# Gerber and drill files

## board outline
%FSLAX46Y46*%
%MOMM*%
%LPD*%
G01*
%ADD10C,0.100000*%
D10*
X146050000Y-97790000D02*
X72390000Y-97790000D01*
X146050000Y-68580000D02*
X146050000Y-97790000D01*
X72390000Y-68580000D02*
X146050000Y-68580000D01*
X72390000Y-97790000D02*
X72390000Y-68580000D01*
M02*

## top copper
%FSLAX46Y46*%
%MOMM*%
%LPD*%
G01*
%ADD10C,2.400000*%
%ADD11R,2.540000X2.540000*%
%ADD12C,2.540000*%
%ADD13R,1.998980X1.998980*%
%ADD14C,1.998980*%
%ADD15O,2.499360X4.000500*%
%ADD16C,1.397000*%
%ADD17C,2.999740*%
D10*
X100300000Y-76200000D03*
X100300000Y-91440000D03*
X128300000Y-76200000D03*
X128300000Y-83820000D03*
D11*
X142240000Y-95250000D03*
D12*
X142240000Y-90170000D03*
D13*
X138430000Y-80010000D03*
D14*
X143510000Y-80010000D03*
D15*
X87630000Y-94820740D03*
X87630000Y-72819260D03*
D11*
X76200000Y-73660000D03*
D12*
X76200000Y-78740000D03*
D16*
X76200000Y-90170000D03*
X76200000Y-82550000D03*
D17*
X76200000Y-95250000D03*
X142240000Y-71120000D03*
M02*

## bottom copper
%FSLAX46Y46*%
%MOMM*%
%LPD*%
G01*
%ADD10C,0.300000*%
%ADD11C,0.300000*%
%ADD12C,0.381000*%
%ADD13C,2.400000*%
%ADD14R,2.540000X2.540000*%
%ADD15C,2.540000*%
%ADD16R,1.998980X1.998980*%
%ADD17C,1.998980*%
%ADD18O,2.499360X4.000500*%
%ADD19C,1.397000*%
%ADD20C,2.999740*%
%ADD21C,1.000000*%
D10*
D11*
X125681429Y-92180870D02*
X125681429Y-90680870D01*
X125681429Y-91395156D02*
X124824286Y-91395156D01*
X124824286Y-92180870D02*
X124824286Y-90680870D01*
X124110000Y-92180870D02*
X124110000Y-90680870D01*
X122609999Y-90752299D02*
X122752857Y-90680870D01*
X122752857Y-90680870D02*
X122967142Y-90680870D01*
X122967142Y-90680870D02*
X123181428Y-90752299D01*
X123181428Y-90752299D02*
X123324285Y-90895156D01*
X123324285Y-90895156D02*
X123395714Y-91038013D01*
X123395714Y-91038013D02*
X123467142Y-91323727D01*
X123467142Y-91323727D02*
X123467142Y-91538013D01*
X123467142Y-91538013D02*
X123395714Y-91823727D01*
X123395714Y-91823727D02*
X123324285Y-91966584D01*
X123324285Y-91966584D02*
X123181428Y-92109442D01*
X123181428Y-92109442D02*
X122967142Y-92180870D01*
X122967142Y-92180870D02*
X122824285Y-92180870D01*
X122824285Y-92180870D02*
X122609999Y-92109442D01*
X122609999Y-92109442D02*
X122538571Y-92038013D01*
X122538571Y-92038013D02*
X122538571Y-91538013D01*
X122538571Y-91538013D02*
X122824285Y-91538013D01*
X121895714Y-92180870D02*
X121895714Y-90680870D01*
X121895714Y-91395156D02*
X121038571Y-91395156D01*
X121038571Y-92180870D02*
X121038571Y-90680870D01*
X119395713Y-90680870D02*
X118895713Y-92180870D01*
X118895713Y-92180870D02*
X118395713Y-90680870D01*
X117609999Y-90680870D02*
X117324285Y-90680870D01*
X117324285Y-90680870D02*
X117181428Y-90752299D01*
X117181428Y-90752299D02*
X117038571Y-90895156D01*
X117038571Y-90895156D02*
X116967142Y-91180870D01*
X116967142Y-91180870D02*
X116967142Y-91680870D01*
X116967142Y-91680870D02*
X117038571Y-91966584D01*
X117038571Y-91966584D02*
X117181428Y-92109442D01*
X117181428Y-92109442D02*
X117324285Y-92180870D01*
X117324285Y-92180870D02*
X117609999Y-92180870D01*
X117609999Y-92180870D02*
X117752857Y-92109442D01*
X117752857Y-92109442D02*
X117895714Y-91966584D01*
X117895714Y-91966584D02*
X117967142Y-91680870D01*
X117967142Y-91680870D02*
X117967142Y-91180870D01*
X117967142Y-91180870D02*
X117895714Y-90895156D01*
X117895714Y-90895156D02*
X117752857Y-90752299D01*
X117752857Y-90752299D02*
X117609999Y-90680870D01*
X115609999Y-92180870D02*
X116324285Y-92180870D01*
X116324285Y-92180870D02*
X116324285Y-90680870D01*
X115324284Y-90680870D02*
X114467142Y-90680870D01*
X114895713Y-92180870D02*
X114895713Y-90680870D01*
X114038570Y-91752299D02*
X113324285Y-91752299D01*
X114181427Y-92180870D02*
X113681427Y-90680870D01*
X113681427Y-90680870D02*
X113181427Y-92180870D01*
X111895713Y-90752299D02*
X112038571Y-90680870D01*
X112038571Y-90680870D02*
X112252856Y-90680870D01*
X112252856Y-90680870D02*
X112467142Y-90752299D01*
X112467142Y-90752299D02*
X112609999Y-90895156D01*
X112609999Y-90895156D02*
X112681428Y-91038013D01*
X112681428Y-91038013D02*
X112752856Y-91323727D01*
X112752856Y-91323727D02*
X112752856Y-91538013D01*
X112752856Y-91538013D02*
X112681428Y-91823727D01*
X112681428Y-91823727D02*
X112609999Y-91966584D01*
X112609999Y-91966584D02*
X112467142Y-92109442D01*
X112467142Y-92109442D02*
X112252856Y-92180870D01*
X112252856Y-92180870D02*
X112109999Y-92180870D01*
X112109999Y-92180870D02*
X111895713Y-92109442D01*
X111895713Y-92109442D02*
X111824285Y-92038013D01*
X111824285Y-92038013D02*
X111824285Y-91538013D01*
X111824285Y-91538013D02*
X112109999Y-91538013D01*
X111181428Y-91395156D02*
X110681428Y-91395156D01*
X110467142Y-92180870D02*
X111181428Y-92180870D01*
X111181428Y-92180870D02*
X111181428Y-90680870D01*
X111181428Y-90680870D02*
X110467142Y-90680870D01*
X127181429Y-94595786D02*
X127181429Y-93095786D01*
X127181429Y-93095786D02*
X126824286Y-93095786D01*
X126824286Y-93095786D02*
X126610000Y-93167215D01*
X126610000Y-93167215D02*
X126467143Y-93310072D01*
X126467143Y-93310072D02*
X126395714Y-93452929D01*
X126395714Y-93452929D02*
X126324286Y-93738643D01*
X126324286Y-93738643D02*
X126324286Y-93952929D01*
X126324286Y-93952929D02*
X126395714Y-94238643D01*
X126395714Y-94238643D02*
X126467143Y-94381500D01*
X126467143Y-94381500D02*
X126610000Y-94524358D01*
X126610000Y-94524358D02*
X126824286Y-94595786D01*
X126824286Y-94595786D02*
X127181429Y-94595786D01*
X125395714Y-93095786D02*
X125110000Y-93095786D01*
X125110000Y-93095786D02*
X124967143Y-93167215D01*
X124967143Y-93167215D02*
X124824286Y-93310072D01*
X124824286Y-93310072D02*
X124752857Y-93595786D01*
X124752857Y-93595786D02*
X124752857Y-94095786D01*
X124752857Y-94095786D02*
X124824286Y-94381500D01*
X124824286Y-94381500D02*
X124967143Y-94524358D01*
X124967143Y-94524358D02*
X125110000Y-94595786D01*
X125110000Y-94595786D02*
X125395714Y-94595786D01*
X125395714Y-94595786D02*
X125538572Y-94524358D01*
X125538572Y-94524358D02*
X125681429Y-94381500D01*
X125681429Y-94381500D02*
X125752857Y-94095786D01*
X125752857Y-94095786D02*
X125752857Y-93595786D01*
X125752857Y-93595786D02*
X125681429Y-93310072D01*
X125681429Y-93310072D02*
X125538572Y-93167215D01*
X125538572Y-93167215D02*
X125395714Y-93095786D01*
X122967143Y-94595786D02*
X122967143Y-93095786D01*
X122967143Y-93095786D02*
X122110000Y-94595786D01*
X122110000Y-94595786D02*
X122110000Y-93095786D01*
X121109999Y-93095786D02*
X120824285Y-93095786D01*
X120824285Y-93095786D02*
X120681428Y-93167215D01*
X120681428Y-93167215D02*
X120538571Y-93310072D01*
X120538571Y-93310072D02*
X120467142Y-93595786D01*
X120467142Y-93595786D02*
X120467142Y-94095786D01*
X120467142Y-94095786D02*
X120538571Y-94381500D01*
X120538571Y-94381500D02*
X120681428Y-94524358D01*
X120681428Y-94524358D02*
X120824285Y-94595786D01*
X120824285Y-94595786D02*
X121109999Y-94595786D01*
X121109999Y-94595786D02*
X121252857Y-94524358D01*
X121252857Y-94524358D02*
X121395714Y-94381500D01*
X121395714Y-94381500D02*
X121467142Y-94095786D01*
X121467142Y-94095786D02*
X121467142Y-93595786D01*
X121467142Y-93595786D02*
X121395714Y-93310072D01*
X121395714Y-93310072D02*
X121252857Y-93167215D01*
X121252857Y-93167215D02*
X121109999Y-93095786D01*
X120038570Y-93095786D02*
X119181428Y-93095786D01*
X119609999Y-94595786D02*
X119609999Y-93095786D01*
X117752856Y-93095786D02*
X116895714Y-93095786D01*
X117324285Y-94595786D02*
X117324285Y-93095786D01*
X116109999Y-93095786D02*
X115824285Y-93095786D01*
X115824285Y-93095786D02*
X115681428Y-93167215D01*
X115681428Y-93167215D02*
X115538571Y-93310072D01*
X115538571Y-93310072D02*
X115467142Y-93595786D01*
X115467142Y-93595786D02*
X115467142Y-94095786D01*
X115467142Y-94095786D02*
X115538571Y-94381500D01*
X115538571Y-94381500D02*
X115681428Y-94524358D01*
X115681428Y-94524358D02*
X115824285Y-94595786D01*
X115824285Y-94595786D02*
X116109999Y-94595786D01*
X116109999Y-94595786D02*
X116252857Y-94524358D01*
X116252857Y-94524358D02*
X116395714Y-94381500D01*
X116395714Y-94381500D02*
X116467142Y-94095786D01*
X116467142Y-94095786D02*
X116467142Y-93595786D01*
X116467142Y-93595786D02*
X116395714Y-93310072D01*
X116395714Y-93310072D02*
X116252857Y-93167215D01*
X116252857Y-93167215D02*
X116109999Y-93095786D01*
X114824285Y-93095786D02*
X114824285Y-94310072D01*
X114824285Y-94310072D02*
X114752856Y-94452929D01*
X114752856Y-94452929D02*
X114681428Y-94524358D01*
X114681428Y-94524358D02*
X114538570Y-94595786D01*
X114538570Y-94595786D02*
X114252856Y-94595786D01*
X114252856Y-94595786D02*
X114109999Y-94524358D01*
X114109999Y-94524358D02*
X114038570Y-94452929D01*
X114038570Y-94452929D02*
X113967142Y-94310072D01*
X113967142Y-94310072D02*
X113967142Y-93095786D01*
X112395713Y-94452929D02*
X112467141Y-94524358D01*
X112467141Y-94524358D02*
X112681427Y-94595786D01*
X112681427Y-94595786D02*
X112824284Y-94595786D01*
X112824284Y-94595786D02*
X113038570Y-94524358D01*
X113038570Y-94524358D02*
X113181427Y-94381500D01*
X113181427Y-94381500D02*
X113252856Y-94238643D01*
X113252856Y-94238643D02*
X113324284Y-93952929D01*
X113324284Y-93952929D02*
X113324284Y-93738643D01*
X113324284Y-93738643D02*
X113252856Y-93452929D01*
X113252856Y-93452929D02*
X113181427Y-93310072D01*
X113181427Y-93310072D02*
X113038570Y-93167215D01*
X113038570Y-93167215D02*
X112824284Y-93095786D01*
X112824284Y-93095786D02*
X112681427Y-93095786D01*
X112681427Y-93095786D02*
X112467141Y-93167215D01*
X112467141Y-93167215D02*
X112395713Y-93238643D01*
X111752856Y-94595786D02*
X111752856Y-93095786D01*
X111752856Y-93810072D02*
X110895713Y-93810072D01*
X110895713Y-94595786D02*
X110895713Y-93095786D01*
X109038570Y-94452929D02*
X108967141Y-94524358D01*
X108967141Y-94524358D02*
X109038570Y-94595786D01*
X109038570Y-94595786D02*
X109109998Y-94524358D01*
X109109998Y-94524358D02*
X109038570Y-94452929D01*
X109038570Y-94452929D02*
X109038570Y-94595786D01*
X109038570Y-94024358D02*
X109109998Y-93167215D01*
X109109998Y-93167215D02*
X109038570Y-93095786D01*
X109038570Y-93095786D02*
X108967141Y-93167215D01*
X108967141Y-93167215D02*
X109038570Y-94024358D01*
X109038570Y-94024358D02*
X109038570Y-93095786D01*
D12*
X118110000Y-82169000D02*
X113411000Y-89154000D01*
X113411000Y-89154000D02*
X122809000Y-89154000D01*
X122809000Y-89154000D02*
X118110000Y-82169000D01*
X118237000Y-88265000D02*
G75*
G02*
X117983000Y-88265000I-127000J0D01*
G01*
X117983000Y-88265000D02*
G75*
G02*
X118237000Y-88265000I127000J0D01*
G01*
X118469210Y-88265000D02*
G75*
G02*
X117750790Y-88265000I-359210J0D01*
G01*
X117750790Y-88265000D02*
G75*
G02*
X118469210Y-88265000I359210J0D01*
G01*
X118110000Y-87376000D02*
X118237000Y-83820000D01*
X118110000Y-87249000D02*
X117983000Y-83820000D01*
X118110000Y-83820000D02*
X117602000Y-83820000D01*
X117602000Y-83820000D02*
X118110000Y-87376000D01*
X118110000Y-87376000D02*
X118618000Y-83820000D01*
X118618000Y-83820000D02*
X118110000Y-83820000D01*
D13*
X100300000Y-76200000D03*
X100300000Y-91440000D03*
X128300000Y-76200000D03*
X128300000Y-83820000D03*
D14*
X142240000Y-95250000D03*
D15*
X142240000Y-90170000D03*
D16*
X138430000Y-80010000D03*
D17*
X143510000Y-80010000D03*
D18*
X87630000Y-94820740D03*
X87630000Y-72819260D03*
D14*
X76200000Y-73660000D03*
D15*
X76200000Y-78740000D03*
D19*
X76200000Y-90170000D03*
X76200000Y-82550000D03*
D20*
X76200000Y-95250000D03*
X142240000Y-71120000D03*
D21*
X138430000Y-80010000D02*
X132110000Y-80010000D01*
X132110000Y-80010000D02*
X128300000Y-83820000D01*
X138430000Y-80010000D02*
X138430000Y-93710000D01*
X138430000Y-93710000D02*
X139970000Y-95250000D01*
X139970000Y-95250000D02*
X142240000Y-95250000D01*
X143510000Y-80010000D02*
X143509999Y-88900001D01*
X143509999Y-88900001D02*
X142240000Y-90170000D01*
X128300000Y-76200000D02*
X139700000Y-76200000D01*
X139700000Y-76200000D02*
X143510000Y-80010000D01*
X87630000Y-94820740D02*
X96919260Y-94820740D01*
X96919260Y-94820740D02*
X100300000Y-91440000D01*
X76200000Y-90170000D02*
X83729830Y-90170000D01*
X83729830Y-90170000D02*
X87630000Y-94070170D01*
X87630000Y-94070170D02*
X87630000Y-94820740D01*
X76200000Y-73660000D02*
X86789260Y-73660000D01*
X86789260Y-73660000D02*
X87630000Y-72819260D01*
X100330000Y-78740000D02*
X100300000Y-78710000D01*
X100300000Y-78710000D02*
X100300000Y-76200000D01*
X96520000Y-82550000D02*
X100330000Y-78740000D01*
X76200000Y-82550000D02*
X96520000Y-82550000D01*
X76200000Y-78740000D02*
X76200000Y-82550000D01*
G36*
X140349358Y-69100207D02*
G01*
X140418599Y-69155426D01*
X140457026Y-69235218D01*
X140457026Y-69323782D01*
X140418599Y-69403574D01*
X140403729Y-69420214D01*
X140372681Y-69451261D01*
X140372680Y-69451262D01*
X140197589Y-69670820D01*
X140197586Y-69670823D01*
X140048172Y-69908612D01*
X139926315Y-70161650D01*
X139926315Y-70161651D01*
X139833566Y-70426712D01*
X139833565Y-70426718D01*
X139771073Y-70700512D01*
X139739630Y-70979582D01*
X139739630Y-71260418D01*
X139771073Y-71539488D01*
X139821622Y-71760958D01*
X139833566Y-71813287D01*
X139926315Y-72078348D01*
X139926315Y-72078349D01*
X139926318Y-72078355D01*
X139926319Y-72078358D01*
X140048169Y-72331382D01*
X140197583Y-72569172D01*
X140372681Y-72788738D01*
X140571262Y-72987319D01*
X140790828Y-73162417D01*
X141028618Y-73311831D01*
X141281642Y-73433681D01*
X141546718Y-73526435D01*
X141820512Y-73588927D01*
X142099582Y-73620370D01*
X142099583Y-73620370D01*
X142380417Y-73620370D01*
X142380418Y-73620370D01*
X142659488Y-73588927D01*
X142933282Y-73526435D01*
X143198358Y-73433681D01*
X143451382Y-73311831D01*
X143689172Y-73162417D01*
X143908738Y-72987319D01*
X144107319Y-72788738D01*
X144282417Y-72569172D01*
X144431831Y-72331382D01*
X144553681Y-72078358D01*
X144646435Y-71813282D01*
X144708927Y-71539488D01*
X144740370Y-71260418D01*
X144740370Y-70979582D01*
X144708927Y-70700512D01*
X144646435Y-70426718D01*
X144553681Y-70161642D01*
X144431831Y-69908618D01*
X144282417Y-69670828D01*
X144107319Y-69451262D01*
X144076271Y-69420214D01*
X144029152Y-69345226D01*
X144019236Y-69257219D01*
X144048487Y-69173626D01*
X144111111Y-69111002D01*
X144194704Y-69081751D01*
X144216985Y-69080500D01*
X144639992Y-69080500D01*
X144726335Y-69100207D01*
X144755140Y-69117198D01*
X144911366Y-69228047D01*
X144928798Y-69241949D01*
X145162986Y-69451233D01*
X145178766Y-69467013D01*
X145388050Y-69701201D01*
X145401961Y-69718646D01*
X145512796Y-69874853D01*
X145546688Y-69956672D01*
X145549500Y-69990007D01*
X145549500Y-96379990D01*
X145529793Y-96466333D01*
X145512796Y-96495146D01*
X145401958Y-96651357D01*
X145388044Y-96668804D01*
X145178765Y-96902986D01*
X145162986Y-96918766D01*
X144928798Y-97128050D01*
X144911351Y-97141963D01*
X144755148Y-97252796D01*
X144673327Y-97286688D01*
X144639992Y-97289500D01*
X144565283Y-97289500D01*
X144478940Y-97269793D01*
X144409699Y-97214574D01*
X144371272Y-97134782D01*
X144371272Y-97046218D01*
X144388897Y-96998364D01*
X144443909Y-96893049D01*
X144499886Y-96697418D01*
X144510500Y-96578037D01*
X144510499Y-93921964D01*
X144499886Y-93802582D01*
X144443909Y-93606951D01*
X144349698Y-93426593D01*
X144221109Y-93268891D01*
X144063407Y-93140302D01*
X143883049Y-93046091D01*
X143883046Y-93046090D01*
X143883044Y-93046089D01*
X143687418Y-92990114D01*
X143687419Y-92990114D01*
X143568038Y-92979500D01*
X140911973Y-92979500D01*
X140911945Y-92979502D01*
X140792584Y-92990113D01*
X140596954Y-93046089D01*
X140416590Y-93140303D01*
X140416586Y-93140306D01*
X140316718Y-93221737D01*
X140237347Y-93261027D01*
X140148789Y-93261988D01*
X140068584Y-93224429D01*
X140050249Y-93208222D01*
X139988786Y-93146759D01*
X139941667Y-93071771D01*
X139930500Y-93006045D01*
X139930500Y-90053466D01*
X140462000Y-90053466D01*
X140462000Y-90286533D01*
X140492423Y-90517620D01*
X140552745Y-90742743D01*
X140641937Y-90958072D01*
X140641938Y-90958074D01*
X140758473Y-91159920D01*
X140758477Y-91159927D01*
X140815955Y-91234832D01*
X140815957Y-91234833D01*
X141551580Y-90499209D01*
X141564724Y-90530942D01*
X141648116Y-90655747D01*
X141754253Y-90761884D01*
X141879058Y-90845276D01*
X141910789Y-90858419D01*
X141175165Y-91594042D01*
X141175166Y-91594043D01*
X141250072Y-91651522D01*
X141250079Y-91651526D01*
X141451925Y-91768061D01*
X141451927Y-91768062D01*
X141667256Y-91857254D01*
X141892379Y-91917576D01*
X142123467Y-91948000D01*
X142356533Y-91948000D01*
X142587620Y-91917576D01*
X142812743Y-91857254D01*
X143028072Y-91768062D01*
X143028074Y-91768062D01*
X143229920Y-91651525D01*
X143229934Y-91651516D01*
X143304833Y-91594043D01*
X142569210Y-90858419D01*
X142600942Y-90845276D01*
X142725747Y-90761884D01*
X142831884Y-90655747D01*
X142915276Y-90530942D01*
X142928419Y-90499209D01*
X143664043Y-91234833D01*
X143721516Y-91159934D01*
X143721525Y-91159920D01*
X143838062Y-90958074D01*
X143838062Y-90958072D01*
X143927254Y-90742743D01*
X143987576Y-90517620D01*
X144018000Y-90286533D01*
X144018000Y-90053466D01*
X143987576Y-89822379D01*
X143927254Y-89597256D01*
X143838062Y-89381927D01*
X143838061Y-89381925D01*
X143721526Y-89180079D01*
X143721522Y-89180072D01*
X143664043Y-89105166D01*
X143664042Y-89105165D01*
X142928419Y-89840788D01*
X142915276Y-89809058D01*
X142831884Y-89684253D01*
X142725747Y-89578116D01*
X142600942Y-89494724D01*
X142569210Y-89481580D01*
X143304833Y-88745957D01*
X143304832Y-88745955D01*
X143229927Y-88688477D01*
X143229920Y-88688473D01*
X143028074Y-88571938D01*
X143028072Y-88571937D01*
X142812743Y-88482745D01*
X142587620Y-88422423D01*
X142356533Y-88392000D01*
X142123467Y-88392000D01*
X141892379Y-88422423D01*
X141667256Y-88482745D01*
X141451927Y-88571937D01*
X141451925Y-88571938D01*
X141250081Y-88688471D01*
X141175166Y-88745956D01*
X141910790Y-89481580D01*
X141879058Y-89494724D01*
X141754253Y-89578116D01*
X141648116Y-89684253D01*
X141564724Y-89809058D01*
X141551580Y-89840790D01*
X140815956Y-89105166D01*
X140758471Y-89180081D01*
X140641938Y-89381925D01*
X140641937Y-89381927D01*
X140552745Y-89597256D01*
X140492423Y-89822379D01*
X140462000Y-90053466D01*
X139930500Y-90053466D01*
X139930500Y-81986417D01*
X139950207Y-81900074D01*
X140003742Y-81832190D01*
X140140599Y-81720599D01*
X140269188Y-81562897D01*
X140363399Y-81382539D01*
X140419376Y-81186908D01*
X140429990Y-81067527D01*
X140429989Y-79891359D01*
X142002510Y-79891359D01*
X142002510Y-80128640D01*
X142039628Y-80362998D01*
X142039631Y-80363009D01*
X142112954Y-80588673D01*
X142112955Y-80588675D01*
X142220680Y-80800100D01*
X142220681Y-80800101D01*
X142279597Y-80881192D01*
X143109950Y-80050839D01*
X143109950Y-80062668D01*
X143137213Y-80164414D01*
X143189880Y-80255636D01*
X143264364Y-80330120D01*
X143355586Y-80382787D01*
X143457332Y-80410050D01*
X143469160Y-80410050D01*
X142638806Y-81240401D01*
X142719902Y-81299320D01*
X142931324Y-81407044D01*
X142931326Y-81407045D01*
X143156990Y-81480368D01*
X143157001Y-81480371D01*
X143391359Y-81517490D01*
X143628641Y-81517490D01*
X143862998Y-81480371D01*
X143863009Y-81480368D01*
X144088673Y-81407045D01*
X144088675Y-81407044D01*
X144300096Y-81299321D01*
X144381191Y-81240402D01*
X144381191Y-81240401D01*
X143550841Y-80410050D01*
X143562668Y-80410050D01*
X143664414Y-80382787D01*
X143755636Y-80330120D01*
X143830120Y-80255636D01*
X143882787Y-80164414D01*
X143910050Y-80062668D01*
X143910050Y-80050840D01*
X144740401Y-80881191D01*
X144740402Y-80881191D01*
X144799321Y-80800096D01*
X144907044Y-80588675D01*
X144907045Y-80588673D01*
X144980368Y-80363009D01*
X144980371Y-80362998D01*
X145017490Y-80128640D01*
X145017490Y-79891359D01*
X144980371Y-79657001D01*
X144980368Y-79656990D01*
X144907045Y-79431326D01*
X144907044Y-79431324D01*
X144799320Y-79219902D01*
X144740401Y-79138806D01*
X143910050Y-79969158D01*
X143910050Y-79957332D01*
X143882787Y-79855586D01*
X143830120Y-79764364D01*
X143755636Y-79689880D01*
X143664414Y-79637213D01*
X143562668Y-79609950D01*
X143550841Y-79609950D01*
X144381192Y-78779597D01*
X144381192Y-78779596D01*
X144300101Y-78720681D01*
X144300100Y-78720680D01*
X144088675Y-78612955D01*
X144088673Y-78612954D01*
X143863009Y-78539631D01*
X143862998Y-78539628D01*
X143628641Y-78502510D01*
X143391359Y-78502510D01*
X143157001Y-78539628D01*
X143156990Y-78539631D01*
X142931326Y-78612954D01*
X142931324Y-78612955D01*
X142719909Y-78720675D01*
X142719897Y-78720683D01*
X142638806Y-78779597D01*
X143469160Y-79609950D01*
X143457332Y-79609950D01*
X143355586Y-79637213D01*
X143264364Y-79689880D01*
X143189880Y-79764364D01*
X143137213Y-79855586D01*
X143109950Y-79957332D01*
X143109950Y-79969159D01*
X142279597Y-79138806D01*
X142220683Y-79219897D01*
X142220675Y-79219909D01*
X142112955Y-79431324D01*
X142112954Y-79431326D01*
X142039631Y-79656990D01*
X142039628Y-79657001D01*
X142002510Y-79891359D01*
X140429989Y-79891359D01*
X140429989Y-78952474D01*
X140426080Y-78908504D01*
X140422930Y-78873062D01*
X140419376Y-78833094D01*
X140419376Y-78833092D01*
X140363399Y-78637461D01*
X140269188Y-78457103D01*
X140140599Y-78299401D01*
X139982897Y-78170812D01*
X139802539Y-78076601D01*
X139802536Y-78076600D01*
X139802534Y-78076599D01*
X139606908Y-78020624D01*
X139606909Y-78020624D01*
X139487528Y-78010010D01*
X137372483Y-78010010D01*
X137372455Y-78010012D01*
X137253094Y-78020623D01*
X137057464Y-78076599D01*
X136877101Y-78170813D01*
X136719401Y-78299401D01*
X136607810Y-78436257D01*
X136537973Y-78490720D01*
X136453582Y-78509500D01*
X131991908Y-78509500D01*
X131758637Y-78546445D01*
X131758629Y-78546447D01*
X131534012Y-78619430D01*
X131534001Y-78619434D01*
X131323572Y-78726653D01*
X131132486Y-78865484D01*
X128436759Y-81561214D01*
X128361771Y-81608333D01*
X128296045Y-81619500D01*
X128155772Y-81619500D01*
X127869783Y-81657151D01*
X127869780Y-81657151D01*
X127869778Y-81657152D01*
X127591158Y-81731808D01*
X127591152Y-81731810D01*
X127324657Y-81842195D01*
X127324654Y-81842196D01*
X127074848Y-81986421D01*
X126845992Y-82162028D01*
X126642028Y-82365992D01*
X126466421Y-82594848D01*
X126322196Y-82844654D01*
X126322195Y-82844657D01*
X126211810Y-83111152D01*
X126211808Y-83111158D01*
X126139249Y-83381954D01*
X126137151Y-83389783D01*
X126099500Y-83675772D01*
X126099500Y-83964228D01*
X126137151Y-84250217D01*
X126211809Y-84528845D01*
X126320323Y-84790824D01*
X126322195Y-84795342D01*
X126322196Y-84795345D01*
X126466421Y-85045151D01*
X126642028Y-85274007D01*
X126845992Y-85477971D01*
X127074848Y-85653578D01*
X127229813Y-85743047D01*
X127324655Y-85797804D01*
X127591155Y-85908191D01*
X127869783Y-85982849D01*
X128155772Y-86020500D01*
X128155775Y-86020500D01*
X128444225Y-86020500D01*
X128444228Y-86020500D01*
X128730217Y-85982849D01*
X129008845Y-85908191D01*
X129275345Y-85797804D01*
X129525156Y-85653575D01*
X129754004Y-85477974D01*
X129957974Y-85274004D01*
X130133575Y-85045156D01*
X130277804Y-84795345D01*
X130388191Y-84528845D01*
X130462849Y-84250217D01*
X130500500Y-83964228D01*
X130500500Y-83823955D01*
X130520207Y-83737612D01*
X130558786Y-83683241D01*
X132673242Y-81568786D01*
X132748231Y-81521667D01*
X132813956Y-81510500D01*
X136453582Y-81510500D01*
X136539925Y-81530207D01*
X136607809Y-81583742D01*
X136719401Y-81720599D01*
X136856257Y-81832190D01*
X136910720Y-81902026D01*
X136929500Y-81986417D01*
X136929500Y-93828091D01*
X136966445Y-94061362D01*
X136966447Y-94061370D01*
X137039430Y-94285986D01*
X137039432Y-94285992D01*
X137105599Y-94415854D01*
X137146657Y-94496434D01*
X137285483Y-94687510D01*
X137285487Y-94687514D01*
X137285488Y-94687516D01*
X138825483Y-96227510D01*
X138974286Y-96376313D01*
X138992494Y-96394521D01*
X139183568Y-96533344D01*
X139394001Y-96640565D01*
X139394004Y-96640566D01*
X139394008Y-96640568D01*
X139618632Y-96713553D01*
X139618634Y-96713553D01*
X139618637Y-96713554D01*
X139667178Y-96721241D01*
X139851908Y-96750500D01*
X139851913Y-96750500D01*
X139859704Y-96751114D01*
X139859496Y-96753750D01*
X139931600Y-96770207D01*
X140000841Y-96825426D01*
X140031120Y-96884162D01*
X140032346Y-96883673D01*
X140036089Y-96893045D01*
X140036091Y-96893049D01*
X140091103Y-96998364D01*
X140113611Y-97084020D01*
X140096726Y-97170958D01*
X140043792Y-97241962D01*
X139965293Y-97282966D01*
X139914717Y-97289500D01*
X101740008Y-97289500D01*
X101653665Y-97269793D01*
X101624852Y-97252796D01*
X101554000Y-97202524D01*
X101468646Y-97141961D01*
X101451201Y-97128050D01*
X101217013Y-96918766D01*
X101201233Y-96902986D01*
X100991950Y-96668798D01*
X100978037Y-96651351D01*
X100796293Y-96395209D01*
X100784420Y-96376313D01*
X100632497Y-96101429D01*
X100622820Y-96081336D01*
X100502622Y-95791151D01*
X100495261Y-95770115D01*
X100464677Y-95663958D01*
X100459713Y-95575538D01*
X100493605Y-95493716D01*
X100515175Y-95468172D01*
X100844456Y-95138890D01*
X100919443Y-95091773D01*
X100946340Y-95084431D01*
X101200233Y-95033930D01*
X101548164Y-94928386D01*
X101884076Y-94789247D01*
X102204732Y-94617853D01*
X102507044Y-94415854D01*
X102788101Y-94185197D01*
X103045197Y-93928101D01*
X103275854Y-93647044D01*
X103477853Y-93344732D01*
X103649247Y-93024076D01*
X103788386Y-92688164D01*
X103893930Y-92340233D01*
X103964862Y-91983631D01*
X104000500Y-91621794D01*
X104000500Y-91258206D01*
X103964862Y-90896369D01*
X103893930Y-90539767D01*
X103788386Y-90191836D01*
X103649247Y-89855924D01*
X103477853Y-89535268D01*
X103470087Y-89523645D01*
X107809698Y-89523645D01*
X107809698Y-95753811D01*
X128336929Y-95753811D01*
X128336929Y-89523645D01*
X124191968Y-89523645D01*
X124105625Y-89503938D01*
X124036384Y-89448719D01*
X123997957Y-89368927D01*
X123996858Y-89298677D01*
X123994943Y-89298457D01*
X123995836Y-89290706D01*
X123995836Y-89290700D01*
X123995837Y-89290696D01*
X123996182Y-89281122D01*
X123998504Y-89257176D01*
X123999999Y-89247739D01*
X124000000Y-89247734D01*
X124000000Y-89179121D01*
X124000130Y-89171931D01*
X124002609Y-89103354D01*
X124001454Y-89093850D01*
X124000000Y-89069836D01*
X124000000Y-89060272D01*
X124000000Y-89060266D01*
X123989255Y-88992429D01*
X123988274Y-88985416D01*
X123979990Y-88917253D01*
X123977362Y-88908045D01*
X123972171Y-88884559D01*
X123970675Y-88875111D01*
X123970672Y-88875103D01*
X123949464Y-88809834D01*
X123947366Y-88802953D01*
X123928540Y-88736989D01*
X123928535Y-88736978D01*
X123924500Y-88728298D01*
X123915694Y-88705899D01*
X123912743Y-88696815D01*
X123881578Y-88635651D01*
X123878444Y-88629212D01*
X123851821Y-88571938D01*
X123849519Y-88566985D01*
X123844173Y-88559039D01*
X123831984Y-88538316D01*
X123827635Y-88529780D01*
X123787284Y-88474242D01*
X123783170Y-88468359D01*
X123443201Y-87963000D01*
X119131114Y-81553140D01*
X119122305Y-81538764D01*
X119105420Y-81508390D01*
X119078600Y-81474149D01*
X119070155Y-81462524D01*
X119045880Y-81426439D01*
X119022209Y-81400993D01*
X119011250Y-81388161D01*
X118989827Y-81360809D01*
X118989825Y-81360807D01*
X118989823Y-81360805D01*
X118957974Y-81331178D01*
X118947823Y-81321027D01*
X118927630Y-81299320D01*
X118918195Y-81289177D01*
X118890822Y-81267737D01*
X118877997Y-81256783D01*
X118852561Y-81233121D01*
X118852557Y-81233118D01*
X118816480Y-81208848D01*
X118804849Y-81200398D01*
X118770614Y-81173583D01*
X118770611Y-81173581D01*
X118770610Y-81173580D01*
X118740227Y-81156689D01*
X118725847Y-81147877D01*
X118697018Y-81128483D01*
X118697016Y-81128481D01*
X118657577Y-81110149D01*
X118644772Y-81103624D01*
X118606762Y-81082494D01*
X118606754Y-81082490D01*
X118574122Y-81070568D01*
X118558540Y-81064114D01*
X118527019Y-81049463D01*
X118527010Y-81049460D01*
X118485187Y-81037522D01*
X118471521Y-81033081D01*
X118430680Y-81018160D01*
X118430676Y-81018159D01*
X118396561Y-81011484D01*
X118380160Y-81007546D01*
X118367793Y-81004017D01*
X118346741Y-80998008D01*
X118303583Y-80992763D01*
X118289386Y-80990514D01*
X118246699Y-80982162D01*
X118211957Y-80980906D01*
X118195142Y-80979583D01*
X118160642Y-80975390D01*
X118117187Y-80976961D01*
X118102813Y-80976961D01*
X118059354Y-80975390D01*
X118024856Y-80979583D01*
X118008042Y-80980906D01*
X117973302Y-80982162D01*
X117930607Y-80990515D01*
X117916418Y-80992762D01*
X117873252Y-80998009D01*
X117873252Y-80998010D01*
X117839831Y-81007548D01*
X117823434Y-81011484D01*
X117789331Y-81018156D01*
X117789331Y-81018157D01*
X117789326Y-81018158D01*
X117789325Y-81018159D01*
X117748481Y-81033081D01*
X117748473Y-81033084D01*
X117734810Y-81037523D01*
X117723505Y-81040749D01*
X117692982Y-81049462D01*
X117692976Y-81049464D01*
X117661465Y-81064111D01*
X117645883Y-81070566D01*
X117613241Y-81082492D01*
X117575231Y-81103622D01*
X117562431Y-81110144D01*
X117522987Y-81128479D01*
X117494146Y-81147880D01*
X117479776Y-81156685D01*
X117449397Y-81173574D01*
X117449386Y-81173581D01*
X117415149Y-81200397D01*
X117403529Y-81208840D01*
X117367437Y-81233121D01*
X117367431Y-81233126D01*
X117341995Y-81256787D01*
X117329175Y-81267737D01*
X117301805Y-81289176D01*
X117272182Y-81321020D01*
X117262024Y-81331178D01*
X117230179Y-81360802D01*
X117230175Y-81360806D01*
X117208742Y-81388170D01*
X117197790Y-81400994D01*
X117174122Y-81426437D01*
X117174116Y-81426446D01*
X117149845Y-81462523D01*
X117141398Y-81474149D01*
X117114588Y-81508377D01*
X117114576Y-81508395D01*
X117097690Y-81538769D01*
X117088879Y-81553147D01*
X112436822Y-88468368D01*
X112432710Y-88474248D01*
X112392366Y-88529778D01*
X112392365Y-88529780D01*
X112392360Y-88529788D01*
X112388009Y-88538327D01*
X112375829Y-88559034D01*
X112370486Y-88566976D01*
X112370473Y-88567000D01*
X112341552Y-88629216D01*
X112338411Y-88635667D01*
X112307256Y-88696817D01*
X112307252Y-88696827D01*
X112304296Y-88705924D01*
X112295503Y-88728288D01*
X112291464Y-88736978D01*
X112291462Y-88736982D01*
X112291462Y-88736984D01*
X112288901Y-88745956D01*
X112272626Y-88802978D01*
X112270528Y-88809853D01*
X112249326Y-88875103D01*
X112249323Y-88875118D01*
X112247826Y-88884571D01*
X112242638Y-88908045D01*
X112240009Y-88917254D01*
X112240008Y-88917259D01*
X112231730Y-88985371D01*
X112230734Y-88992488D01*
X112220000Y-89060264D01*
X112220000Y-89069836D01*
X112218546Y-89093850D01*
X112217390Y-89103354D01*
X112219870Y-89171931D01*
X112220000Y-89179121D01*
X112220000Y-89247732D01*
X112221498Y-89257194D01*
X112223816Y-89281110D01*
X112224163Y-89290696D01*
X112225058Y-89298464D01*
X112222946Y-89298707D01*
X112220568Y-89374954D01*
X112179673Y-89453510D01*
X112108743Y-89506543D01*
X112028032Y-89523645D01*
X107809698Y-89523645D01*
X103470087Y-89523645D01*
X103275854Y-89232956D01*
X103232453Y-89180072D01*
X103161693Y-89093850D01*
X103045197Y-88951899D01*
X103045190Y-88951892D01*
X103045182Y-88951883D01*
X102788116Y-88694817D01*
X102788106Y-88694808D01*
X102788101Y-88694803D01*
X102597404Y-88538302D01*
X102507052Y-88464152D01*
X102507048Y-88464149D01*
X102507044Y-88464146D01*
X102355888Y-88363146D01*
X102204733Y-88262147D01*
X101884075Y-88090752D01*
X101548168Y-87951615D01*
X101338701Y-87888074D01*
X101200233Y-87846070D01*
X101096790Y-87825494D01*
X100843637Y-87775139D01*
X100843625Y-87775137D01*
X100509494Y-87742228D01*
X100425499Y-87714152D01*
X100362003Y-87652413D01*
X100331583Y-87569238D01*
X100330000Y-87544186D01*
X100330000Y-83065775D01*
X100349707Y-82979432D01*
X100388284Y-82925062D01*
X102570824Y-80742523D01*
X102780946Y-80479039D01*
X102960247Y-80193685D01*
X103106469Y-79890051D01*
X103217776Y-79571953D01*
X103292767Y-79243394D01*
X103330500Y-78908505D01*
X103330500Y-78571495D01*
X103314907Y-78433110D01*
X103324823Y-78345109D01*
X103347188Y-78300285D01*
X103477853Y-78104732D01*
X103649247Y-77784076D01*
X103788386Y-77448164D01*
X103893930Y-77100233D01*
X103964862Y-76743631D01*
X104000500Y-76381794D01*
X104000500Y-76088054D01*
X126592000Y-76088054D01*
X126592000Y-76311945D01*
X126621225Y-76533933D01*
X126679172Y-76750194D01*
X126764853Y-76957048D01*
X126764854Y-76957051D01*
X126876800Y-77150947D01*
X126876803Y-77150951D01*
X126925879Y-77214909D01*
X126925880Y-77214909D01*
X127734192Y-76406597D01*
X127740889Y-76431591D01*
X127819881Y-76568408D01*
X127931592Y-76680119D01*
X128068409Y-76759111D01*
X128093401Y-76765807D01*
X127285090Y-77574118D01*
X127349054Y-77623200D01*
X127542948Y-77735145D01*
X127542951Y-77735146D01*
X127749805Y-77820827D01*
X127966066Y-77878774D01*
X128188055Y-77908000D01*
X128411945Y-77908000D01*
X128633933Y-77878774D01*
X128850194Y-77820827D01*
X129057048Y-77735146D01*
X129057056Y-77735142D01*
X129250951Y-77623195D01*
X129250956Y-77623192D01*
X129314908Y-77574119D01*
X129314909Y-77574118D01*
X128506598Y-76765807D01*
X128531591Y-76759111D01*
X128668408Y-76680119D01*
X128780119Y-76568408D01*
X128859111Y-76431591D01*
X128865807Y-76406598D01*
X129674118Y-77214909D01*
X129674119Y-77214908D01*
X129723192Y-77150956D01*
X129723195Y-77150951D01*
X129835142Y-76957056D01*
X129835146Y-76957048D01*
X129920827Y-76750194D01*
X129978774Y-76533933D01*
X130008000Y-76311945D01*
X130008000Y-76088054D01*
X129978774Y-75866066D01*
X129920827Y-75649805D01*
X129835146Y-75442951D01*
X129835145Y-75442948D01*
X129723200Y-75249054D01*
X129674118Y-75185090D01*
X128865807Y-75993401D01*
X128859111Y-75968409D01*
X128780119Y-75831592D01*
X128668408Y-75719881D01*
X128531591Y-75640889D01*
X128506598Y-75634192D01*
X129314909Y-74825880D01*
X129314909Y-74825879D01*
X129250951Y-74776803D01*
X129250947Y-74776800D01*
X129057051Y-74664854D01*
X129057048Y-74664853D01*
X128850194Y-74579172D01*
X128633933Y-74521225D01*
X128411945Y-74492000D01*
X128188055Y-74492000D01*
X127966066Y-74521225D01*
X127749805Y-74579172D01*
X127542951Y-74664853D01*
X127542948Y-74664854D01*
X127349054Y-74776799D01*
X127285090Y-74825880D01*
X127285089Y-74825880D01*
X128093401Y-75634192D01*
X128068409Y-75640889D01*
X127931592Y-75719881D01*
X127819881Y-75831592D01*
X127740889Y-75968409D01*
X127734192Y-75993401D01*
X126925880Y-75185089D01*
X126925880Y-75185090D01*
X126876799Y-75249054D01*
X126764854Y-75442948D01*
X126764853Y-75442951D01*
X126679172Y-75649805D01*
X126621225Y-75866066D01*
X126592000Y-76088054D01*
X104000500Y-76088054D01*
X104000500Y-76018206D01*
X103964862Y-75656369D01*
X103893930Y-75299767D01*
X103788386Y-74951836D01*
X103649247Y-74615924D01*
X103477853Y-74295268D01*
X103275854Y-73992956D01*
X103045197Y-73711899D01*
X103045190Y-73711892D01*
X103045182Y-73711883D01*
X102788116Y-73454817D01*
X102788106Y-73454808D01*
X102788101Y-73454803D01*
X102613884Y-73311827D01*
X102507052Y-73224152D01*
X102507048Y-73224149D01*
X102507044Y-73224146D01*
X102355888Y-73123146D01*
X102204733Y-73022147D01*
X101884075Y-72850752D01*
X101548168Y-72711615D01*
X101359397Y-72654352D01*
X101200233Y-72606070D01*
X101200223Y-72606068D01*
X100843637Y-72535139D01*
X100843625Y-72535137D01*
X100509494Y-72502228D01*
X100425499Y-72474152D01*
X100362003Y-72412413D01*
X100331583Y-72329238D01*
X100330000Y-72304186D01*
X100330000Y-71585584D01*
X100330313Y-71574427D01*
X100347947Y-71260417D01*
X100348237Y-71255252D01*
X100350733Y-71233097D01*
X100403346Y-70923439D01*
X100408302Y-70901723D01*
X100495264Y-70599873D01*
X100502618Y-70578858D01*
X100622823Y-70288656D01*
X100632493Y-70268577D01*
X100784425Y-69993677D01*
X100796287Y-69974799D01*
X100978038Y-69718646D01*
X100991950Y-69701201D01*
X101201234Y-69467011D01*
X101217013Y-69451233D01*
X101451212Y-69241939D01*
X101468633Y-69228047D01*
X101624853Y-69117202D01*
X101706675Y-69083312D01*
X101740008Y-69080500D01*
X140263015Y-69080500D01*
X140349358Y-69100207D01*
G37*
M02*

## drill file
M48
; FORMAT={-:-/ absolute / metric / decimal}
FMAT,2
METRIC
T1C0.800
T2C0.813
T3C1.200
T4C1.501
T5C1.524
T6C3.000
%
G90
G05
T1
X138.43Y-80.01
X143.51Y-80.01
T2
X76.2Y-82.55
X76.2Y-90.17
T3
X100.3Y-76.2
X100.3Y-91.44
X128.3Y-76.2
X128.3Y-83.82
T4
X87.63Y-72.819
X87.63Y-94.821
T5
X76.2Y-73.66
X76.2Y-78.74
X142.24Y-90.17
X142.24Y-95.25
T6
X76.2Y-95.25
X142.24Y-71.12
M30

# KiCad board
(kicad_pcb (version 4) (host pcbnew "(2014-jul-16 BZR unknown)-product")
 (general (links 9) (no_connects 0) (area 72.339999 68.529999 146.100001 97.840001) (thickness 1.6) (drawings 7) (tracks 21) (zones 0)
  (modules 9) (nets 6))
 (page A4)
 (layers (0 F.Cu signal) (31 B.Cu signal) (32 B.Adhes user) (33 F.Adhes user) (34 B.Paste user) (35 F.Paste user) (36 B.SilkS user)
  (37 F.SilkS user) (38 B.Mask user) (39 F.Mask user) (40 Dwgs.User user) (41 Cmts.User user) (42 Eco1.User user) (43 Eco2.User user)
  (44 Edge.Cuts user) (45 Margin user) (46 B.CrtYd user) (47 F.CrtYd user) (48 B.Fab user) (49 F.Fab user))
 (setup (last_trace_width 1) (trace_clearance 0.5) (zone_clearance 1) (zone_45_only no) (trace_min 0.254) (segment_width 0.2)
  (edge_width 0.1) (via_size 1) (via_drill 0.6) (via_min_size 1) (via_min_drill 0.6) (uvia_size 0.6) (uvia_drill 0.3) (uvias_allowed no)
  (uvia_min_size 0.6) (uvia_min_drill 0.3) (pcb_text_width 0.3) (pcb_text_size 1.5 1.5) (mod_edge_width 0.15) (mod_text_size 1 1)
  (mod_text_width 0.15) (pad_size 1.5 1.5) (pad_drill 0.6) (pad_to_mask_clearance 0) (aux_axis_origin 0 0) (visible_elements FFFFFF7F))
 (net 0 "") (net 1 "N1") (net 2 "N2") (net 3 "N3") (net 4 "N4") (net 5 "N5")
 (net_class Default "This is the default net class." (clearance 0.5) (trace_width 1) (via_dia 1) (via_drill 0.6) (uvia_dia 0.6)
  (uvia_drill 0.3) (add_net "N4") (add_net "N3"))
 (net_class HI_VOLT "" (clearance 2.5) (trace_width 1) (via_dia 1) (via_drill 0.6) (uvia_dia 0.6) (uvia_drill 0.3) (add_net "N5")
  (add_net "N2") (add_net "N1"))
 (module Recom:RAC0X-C (layer F.Cu) (at 114.3 83.82)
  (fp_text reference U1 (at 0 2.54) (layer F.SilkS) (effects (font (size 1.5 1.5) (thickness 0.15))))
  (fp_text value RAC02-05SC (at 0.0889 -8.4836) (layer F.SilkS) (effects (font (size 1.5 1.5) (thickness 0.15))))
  (pad 1 thru_hole circle (at -14 -7.62) (size 2.4 2.4) (drill 1.2) (layers *.Cu *.Mask F.SilkS) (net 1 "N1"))
  (pad 2 thru_hole circle (at -14 7.62) (size 2.4 2.4) (drill 1.2) (layers *.Cu *.Mask F.SilkS) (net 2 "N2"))
  (pad 3 thru_hole circle (at 14 -7.62) (size 2.4 2.4) (drill 1.2) (layers *.Cu *.Mask F.SilkS) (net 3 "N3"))
  (pad 4 thru_hole circle (at 14 0) (size 2.4 2.4) (drill 1.2) (layers *.Cu *.Mask F.SilkS) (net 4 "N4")))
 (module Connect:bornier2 (layer F.Cu) (at 142.24 92.71 90)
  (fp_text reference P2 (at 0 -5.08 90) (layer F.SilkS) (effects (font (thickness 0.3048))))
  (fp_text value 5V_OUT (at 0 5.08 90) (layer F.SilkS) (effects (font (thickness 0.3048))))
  (pad 1 thru_hole rect (at -2.54 0 90) (size 2.54 2.54) (drill 1.524) (layers *.Cu *.Mask F.SilkS) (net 4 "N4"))
  (pad 2 thru_hole circle (at 2.54 0 90) (size 2.54 2.54) (drill 1.524) (layers *.Cu *.Mask F.SilkS) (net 3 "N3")))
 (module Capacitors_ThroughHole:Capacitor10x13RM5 (layer F.Cu) (at 140.97 80.01 270)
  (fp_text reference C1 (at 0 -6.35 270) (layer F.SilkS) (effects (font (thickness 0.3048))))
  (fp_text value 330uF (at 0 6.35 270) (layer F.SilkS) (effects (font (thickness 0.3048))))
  (pad 1 thru_hole rect (at 0 2.54 270) (size 1.99898 1.99898) (drill 0.8001) (layers *.Cu *.Mask F.SilkS) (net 4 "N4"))
  (pad 2 thru_hole circle (at 0 -2.54 270) (size 1.99898 1.99898) (drill 0.8001) (layers *.Cu *.Mask F.SilkS) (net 3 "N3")))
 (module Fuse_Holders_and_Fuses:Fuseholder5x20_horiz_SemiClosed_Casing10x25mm (layer F.Cu) (at 87.63 83.82 270)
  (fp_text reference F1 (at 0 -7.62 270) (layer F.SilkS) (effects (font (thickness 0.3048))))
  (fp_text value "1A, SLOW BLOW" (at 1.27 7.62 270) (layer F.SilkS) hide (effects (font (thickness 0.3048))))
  (pad 2 thru_hole oval (at 11.00074 0 180) (size 2.49936 4.0005) (drill 1.50114) (layers *.Cu *.Mask F.SilkS) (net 2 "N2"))
  (pad 1 thru_hole oval (at -11.00074 0 180) (size 2.49936 4.0005) (drill 1.50114) (layers *.Cu *.Mask F.SilkS) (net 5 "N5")))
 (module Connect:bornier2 (layer F.Cu) (at 76.2 76.2 270)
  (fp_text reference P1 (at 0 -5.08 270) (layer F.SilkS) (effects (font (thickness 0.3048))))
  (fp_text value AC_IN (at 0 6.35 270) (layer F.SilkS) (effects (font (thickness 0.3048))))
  (pad 1 thru_hole rect (at -2.54 0 270) (size 2.54 2.54) (drill 1.524) (layers *.Cu *.Mask F.SilkS) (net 5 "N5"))
  (pad 2 thru_hole circle (at 2.54 0 270) (size 2.54 2.54) (drill 1.524) (layers *.Cu *.Mask F.SilkS) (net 1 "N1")))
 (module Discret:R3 (layer F.Cu) (at 76.2 86.36 90) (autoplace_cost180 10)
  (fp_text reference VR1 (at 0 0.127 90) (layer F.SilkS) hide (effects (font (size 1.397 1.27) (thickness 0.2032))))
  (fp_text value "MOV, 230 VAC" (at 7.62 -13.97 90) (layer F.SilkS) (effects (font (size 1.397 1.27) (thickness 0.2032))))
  (pad 1 thru_hole circle (at -3.81 0 90) (size 1.397 1.397) (drill 0.8128) (layers *.Cu *.Mask F.SilkS) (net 2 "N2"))
  (pad 2 thru_hole circle (at 3.81 0 90) (size 1.397 1.397) (drill 0.8128) (layers *.Cu *.Mask F.SilkS) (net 1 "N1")))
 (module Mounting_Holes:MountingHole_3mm (layer F.Cu) (at 76.2 95.25)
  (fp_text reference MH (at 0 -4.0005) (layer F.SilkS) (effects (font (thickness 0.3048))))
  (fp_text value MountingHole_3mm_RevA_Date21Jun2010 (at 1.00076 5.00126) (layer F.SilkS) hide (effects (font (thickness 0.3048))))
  (pad 1 thru_hole circle (at 0 0) (size 2.99974 2.99974) (drill 2.99974) (layers)))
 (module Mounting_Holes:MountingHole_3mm (layer F.Cu) (at 142.24 71.12)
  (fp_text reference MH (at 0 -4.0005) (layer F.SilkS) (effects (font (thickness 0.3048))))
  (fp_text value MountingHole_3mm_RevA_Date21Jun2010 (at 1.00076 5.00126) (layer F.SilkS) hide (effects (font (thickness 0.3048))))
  (pad 1 thru_hole circle (at 0 0) (size 2.99974 2.99974) (drill 2.99974) (layers)))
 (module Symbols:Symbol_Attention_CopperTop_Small (layer B.Cu) (at 118.11 86.36 180)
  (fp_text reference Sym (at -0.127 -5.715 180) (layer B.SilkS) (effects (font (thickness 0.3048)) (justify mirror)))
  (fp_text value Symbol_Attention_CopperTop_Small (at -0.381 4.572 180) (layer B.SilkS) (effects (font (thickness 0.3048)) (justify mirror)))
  (fp_line (start 0 4.191) (end 4.699 -2.794) (layer B.Cu) (width 0.381))
  (fp_line (start 4.699 -2.794) (end -4.699 -2.794) (layer B.Cu) (width 0.381))
  (fp_line (start -4.699 -2.794) (end 0 4.191) (layer B.Cu) (width 0.381))
  (fp_circle (center 0 -1.905) (end 0 -2.032) (layer B.Cu) (width 0.381))
  (fp_circle (center 0 -1.905) (end 0.254 -2.159) (layer B.Cu) (width 0.381))
  (fp_line (start 0 -1.016) (end -0.127 2.54) (layer B.Cu) (width 0.381))
  (fp_line (start 0 -0.889) (end 0.127 2.54) (layer B.Cu) (width 0.381))
  (fp_line (start 0 2.54) (end 0.508 2.54) (layer B.Cu) (width 0.381))
  (fp_line (start 0.508 2.54) (end 0 -1.016) (layer B.Cu) (width 0.381))
  (fp_line (start 0 -1.016) (end -0.508 2.54) (layer B.Cu) (width 0.381))
  (fp_line (start -0.508 2.54) (end 0 2.54) (layer B.Cu) (width 0.381)))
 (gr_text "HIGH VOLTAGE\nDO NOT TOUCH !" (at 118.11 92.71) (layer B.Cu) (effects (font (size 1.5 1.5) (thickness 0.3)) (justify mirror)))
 (gr_line (start 146.05 97.79) (end 72.39 97.79) (layer Edge.Cuts) (width 0.1))
 (gr_line (start 146.05 68.58) (end 146.05 97.79) (layer Edge.Cuts) (width 0.1))
 (gr_line (start 72.39 68.58) (end 146.05 68.58) (layer Edge.Cuts) (width 0.1))
 (gr_line (start 72.39 97.79) (end 72.39 68.58) (layer Edge.Cuts) (width 0.1))
 (segment (start 138.43 80.01) (end 132.11 80.01) (width 1) (layer B.Cu) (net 4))
 (segment (start 132.11 80.01) (end 128.3 83.82) (width 1) (layer B.Cu) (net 4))
 (segment (start 138.43 80.01) (end 138.43 93.71) (width 1) (layer B.Cu) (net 4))
 (segment (start 138.43 93.71) (end 139.97 95.25) (width 1) (layer B.Cu) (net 4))
 (segment (start 139.97 95.25) (end 142.24 95.25) (width 1) (layer B.Cu) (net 4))
 (segment (start 143.51 80.01) (end 143.509999 88.900001) (width 1) (layer B.Cu) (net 3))
 (segment (start 143.509999 88.900001) (end 142.24 90.17) (width 1) (layer B.Cu) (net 3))
 (segment (start 128.3 76.2) (end 139.7 76.2) (width 1) (layer B.Cu) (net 3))
 (segment (start 139.7 76.2) (end 143.51 80.01) (width 1) (layer B.Cu) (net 3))
 (segment (start 87.63 94.82074) (end 96.91926 94.82074) (width 1) (layer B.Cu) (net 2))
 (segment (start 96.91926 94.82074) (end 100.3 91.44) (width 1) (layer B.Cu) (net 2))
 (segment (start 76.2 90.17) (end 83.72983 90.17) (width 1) (layer B.Cu) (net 2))
 (segment (start 83.72983 90.17) (end 87.63 94.07017) (width 1) (layer B.Cu) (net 2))
 (segment (start 87.63 94.07017) (end 87.63 94.82074) (width 1) (layer B.Cu) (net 2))
 (segment (start 76.2 73.66) (end 86.78926 73.66) (width 1) (layer B.Cu) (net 5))
 (segment (start 86.78926 73.66) (end 87.63 72.81926) (width 1) (layer B.Cu) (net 5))
 (segment (start 100.33 78.74) (end 100.3 78.71) (width 1) (layer B.Cu) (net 1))
 (segment (start 100.3 78.71) (end 100.3 76.2) (width 1) (layer B.Cu) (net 1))
 (segment (start 96.52 82.55) (end 100.33 78.74) (width 1) (layer B.Cu) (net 1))
 (segment (start 76.2 82.55) (end 96.52 82.55) (width 1) (layer B.Cu) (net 1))
 (segment (start 76.2 78.74) (end 76.2 82.55) (width 1) (layer B.Cu) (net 1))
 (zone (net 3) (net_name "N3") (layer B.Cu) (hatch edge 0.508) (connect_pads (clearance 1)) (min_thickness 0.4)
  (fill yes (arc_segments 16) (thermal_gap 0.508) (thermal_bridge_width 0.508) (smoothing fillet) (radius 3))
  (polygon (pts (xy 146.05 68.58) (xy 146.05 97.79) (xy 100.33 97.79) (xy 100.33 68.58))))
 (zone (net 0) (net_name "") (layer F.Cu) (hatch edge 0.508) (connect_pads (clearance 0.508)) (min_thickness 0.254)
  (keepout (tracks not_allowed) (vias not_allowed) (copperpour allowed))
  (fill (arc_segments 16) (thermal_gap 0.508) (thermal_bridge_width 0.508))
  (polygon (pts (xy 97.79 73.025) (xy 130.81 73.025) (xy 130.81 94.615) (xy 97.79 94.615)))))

